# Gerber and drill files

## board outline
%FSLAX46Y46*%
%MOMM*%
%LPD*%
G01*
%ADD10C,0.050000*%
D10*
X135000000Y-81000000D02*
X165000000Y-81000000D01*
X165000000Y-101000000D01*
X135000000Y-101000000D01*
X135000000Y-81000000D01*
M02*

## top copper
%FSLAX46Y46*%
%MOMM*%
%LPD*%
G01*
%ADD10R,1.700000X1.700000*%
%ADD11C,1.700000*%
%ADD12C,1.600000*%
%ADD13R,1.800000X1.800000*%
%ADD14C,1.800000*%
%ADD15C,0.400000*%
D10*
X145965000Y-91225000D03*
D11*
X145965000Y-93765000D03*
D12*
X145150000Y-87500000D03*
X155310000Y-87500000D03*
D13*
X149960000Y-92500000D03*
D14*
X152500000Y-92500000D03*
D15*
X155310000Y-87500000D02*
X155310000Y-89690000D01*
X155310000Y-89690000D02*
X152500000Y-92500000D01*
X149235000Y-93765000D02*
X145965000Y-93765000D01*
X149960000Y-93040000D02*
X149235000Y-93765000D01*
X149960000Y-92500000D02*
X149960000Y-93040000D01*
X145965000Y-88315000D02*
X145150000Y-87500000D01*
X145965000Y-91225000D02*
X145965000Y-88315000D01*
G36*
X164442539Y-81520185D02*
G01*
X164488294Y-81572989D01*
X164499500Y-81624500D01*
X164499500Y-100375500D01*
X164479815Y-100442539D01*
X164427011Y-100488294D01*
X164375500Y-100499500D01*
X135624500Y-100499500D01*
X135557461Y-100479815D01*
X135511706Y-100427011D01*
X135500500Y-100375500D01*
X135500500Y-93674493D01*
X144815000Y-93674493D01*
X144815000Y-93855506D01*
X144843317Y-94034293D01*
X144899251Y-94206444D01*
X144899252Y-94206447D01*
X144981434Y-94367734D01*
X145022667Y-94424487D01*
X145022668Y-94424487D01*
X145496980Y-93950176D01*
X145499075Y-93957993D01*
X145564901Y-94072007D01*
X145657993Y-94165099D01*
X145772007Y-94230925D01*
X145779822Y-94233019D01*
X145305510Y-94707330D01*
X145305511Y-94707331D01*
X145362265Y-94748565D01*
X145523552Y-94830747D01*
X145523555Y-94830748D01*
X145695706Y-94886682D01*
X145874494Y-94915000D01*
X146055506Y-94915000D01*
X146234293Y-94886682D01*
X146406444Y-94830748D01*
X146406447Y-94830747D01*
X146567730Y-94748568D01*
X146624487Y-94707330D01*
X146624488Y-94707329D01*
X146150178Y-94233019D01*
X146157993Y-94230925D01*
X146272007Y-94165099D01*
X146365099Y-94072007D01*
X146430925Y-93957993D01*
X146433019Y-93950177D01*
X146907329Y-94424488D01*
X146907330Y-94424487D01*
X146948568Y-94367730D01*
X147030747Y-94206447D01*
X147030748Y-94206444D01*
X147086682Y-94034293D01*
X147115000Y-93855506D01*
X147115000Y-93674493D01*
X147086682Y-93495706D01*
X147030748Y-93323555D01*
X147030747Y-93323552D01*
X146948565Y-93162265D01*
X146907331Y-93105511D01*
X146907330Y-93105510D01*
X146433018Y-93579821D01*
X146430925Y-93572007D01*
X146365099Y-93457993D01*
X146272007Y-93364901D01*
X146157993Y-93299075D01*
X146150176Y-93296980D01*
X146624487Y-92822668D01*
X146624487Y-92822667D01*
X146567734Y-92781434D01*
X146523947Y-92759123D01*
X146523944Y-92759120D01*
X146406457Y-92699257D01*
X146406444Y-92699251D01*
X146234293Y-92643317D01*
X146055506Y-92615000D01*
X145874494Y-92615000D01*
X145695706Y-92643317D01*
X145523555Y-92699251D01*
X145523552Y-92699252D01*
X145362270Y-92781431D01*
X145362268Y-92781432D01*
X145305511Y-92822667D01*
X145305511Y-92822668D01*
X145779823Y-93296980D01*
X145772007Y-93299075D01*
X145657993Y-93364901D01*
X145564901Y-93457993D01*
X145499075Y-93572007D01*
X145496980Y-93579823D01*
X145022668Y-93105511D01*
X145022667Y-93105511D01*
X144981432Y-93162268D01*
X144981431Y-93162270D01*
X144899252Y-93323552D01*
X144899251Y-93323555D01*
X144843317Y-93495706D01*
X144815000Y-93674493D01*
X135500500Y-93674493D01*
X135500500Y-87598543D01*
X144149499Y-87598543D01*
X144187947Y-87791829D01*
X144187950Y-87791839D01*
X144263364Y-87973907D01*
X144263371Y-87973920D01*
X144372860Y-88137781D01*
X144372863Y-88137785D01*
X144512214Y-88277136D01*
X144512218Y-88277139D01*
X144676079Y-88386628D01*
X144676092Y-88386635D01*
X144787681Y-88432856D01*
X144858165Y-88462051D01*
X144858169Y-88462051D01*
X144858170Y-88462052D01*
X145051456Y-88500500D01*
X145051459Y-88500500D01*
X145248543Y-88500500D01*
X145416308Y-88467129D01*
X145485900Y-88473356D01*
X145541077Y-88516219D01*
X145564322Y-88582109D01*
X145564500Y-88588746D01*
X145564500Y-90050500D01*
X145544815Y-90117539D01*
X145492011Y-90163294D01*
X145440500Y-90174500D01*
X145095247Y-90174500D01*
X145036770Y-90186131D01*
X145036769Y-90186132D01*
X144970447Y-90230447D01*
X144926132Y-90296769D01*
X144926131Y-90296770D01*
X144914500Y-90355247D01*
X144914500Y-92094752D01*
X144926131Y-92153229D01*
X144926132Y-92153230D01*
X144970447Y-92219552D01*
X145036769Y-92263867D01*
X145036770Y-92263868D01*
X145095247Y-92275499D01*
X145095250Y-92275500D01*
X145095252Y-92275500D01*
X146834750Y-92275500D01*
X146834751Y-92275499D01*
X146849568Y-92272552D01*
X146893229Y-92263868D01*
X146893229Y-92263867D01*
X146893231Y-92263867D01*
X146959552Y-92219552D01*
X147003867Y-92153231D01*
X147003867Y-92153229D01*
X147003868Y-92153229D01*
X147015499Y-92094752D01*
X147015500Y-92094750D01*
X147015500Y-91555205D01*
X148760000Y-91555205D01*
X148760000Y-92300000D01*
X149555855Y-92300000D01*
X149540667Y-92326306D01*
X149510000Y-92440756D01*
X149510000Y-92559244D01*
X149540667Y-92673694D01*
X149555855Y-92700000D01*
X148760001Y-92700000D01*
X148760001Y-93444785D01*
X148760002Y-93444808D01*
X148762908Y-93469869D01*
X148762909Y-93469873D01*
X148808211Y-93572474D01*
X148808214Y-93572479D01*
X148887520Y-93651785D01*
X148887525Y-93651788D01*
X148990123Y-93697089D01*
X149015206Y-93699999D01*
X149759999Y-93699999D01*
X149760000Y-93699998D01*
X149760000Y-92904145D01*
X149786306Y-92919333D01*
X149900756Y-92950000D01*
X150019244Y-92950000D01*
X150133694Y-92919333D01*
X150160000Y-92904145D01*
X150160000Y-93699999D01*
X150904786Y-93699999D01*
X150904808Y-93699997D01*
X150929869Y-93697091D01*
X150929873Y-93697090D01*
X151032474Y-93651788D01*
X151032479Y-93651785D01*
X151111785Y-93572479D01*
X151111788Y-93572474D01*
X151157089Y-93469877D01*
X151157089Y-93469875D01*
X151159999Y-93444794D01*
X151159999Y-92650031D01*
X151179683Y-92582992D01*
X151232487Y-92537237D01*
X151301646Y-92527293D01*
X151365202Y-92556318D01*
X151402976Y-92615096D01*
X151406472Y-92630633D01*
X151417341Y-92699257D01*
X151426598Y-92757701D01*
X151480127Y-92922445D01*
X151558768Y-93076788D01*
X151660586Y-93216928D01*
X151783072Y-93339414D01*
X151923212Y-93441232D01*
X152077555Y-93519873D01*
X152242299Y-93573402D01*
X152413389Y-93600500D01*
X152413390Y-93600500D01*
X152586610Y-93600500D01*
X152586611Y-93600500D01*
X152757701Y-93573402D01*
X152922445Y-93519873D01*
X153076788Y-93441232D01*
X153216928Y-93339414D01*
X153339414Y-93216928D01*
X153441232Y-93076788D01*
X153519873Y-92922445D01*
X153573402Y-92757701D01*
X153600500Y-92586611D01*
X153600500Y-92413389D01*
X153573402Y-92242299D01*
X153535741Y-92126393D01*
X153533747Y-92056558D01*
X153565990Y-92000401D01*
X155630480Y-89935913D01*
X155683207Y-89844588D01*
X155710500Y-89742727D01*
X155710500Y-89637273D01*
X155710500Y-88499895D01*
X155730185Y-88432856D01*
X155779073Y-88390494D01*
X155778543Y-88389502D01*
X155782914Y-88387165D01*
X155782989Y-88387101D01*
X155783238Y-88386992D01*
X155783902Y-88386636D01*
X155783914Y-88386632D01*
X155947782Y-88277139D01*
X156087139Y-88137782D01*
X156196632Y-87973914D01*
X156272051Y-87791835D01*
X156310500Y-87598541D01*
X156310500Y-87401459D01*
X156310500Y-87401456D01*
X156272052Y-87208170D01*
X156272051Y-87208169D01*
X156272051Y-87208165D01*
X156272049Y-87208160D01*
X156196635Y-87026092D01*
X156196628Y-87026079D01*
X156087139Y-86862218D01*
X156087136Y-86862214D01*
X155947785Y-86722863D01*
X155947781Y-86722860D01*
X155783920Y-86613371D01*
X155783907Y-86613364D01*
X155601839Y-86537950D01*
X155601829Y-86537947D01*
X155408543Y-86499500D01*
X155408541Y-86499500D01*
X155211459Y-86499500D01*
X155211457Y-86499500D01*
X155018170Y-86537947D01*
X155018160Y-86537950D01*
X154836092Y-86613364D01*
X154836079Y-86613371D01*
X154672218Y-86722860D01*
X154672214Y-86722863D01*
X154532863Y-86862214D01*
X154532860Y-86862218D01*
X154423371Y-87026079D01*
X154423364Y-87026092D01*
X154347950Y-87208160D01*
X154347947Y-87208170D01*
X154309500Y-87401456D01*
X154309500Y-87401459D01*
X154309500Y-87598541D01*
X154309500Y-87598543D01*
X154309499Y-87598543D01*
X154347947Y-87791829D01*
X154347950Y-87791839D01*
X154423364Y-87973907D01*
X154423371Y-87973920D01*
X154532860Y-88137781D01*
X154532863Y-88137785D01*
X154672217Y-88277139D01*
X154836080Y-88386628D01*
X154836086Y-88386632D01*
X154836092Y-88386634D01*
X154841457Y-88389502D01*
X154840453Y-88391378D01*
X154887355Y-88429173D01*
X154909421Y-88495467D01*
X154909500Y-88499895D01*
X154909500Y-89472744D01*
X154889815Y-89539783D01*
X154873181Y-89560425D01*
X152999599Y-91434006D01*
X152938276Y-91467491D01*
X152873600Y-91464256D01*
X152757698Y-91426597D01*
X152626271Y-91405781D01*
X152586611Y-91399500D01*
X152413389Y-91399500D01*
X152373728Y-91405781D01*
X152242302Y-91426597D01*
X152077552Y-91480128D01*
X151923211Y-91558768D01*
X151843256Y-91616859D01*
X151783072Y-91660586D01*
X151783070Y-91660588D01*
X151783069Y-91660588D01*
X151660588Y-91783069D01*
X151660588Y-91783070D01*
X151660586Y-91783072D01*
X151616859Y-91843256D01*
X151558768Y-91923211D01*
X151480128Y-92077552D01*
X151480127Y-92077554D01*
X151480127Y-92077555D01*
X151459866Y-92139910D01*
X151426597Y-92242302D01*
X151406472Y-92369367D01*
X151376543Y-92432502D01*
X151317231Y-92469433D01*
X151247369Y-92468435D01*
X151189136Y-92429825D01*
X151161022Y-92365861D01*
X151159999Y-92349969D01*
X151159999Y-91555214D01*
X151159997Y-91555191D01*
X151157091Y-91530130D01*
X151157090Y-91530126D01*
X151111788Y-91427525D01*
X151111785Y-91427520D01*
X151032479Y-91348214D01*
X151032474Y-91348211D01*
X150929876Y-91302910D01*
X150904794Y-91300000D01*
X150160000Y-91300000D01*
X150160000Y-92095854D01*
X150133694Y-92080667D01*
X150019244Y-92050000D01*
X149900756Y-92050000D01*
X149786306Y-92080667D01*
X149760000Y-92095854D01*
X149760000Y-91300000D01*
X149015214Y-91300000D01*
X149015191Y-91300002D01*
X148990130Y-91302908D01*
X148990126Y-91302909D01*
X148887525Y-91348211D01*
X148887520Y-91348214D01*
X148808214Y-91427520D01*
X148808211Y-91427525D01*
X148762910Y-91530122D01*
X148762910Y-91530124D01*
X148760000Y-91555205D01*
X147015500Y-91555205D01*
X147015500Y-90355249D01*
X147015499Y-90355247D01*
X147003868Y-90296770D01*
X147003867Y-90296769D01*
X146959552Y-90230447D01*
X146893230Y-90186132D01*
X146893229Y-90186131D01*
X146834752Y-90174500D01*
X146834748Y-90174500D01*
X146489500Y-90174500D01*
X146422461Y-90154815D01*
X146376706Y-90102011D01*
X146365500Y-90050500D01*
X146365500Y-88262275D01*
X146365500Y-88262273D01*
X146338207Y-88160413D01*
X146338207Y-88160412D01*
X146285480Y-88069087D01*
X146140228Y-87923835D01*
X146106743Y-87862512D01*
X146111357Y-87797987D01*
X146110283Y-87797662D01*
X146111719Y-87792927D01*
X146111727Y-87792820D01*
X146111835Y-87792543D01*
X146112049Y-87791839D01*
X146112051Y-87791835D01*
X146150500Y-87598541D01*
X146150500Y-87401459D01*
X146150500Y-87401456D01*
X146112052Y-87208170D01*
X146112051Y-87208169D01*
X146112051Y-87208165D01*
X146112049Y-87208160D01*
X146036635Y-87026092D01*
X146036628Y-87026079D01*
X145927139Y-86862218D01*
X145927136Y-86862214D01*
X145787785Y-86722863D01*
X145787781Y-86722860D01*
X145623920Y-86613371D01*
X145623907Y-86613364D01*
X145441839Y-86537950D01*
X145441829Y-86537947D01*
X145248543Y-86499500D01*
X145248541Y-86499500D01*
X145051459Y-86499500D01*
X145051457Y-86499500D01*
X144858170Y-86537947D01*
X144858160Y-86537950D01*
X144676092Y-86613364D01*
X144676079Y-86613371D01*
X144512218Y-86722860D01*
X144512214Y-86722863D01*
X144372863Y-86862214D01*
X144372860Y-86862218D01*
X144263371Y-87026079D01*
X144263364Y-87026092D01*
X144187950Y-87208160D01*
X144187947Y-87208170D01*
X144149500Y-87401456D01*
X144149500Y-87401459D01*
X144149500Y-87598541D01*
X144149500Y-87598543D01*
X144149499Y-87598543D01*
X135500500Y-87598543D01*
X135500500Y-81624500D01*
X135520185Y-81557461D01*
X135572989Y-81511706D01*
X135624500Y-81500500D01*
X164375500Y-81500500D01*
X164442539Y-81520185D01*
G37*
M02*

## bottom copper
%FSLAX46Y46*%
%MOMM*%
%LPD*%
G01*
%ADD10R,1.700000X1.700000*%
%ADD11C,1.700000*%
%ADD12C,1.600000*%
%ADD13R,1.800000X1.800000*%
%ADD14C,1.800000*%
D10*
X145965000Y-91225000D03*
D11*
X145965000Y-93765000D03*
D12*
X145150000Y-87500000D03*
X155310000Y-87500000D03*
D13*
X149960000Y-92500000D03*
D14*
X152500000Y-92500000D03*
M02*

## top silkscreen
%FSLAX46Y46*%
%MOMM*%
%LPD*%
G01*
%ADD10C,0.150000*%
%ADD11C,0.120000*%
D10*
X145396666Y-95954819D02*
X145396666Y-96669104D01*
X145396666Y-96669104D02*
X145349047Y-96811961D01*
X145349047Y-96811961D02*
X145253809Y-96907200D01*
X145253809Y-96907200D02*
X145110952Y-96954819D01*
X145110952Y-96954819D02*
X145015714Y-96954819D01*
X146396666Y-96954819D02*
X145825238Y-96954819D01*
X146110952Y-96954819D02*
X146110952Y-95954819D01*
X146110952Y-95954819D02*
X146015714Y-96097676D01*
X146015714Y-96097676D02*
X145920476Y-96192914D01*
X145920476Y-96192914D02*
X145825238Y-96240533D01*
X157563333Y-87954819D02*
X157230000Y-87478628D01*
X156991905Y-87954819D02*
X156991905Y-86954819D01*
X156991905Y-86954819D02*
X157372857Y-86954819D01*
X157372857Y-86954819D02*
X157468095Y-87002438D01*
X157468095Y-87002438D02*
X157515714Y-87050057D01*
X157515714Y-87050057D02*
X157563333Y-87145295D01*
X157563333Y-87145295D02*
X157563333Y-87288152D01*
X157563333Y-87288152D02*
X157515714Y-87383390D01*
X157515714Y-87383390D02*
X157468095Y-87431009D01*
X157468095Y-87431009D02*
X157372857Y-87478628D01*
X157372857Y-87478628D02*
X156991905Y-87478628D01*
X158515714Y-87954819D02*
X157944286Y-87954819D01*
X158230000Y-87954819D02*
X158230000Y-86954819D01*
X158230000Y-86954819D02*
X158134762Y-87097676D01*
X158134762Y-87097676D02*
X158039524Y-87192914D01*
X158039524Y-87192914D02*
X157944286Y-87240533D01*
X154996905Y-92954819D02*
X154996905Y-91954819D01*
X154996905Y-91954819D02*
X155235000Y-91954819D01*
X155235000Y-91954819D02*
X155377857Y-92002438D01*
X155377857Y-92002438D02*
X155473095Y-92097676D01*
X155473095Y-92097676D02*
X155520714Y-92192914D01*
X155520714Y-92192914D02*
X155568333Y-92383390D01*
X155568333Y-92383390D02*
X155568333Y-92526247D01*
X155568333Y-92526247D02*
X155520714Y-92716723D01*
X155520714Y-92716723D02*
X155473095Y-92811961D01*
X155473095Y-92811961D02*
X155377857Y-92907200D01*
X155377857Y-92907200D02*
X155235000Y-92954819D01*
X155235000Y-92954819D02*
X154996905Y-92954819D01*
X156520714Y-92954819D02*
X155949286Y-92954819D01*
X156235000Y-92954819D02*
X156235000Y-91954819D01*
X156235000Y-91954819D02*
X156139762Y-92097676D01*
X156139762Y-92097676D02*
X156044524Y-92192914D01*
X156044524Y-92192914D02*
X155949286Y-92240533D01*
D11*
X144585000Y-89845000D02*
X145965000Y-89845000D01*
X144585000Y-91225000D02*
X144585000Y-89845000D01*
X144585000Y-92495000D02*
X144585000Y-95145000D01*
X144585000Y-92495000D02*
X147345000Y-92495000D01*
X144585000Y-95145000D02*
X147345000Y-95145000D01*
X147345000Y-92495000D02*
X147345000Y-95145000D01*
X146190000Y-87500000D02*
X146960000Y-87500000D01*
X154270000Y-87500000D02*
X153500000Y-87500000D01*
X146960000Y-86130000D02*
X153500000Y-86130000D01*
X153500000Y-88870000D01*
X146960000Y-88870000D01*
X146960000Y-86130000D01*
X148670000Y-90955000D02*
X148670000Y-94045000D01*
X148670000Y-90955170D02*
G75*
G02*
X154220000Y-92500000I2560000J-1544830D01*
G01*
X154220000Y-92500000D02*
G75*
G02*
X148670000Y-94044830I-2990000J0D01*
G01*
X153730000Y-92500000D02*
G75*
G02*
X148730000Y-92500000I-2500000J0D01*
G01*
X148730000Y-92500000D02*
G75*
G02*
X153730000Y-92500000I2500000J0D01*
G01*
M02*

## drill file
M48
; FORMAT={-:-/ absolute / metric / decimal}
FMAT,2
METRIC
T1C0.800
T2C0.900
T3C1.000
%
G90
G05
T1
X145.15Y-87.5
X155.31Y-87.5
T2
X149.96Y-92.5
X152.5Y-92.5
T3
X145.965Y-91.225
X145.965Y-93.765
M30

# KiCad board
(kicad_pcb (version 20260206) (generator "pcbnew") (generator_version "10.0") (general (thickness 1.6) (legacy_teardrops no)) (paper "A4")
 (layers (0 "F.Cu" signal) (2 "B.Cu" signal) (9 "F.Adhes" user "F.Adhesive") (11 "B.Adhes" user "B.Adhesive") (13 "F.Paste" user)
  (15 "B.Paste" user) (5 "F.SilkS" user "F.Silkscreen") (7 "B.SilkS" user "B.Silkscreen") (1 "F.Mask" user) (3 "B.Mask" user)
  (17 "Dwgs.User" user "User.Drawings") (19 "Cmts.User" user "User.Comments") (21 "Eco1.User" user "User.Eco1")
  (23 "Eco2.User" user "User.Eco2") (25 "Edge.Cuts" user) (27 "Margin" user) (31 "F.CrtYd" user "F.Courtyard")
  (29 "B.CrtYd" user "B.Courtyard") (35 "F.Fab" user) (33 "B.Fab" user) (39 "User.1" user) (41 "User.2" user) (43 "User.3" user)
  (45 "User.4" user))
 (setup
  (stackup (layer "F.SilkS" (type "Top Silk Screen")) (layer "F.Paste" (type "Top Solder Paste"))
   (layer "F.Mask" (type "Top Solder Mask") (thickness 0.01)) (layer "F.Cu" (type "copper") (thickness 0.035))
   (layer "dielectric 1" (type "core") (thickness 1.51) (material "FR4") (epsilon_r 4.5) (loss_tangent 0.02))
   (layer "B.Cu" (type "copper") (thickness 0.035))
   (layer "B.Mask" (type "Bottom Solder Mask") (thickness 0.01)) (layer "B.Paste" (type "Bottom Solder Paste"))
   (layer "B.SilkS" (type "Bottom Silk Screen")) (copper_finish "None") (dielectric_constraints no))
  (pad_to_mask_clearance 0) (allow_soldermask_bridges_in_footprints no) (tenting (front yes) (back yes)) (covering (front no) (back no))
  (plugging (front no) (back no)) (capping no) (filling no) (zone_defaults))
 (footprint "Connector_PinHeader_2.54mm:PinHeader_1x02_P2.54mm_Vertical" (layer "F.Cu") (at 145.965 91.225)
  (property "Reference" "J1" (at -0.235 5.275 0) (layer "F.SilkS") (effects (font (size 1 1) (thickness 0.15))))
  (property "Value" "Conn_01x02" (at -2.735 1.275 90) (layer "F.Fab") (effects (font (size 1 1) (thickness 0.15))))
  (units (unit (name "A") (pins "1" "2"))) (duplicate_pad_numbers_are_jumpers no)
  (fp_line (start -1.38 -1.38) (end 0 -1.38) (stroke (width 0.12) (type solid)) (layer "F.SilkS"))
  (fp_line (start -1.38 0) (end -1.38 -1.38) (stroke (width 0.12) (type solid)) (layer "F.SilkS"))
  (fp_line (start -1.38 1.27) (end -1.38 3.92) (stroke (width 0.12) (type solid)) (layer "F.SilkS"))
  (fp_line (start -1.38 1.27) (end 1.38 1.27) (stroke (width 0.12) (type solid)) (layer "F.SilkS"))
  (fp_line (start -1.38 3.92) (end 1.38 3.92) (stroke (width 0.12) (type solid)) (layer "F.SilkS"))
  (fp_line (start 1.38 1.27) (end 1.38 3.92) (stroke (width 0.12) (type solid)) (layer "F.SilkS"))
  (pad "1" thru_hole rect (at 0 0) (size 1.7 1.7) (drill 1) (layers "*.Cu" "*.Mask") (remove_unused_layers no) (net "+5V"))
  (pad "2" thru_hole circle (at 0 2.54) (size 1.7 1.7) (drill 1) (layers "*.Cu" "*.Mask") (remove_unused_layers no) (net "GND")))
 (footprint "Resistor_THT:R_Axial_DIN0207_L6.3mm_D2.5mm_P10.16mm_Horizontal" (layer "F.Cu") (at 145.15 87.5)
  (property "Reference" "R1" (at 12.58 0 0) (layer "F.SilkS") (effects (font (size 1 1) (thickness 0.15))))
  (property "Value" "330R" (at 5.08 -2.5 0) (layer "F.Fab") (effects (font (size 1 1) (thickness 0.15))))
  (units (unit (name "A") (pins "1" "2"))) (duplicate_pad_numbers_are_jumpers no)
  (fp_line (start 1.04 0) (end 1.81 0) (stroke (width 0.12) (type solid)) (layer "F.SilkS"))
  (fp_line (start 9.12 0) (end 8.35 0) (stroke (width 0.12) (type solid)) (layer "F.SilkS"))
  (fp_rect (start 1.81 -1.37) (end 8.35 1.37) (stroke (width 0.12) (type solid)) (fill no) (layer "F.SilkS"))
  (pad "1" thru_hole circle (at 0 0) (size 1.6 1.6) (drill 0.8) (layers "*.Cu" "*.Mask") (remove_unused_layers no) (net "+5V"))
  (pad "2" thru_hole circle (at 10.16 0) (size 1.6 1.6) (drill 0.8) (layers "*.Cu" "*.Mask") (remove_unused_layers no) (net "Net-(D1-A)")))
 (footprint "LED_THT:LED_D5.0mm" (layer "F.Cu") (at 149.96 92.5)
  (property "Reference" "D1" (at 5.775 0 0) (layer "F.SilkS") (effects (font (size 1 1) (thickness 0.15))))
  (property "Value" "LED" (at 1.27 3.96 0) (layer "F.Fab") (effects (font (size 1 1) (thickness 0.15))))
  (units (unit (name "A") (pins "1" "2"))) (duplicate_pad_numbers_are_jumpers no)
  (fp_line (start -1.29 -1.545) (end -1.29 1.545) (stroke (width 0.12) (type solid)) (layer "F.SilkS"))
  (fp_arc (start -1.29 -1.54483) (mid 2.071779 -2.880495) (end 4.26 0) (stroke (width 0.12) (type solid)) (layer "F.SilkS"))
  (fp_arc (start 4.26 0) (mid 2.071779 2.880495) (end -1.29 1.54483) (stroke (width 0.12) (type solid)) (layer "F.SilkS"))
  (fp_circle (center 1.27 0) (end 3.77 0) (stroke (width 0.12) (type solid)) (fill no) (layer "F.SilkS"))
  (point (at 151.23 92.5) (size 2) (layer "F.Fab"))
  (pad "1" thru_hole rect (at 0 0) (size 1.8 1.8) (drill 0.9) (layers "*.Cu" "*.Mask") (remove_unused_layers no) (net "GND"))
  (pad "2" thru_hole circle (at 2.54 0) (size 1.8 1.8) (drill 0.9) (layers "*.Cu" "*.Mask") (remove_unused_layers no) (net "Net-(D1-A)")))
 (gr_rect (start 135 81) (end 165 101) (stroke (width 0.05) (type default)) (fill no) (layer "Edge.Cuts"))
 (segment (start 155.31 87.5) (end 155.31 89.69) (width 0.4) (layer "F.Cu") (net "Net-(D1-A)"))
 (segment (start 155.31 89.69) (end 152.5 92.5) (width 0.4) (layer "F.Cu") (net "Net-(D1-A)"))
 (segment (start 149.235 93.765) (end 145.965 93.765) (width 0.4) (layer "F.Cu") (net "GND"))
 (segment (start 149.96 93.04) (end 149.235 93.765) (width 0.4) (layer "F.Cu") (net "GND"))
 (segment (start 149.96 92.5) (end 149.96 93.04) (width 0.4) (layer "F.Cu") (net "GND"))
 (segment (start 145.965 88.315) (end 145.15 87.5) (width 0.4) (layer "F.Cu") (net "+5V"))
 (segment (start 145.965 91.225) (end 145.965 88.315) (width 0.4) (layer "F.Cu") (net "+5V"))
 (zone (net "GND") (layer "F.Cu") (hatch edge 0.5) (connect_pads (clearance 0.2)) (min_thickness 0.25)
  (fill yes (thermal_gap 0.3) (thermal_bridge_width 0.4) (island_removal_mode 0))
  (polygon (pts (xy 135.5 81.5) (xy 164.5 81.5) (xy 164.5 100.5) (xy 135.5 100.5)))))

